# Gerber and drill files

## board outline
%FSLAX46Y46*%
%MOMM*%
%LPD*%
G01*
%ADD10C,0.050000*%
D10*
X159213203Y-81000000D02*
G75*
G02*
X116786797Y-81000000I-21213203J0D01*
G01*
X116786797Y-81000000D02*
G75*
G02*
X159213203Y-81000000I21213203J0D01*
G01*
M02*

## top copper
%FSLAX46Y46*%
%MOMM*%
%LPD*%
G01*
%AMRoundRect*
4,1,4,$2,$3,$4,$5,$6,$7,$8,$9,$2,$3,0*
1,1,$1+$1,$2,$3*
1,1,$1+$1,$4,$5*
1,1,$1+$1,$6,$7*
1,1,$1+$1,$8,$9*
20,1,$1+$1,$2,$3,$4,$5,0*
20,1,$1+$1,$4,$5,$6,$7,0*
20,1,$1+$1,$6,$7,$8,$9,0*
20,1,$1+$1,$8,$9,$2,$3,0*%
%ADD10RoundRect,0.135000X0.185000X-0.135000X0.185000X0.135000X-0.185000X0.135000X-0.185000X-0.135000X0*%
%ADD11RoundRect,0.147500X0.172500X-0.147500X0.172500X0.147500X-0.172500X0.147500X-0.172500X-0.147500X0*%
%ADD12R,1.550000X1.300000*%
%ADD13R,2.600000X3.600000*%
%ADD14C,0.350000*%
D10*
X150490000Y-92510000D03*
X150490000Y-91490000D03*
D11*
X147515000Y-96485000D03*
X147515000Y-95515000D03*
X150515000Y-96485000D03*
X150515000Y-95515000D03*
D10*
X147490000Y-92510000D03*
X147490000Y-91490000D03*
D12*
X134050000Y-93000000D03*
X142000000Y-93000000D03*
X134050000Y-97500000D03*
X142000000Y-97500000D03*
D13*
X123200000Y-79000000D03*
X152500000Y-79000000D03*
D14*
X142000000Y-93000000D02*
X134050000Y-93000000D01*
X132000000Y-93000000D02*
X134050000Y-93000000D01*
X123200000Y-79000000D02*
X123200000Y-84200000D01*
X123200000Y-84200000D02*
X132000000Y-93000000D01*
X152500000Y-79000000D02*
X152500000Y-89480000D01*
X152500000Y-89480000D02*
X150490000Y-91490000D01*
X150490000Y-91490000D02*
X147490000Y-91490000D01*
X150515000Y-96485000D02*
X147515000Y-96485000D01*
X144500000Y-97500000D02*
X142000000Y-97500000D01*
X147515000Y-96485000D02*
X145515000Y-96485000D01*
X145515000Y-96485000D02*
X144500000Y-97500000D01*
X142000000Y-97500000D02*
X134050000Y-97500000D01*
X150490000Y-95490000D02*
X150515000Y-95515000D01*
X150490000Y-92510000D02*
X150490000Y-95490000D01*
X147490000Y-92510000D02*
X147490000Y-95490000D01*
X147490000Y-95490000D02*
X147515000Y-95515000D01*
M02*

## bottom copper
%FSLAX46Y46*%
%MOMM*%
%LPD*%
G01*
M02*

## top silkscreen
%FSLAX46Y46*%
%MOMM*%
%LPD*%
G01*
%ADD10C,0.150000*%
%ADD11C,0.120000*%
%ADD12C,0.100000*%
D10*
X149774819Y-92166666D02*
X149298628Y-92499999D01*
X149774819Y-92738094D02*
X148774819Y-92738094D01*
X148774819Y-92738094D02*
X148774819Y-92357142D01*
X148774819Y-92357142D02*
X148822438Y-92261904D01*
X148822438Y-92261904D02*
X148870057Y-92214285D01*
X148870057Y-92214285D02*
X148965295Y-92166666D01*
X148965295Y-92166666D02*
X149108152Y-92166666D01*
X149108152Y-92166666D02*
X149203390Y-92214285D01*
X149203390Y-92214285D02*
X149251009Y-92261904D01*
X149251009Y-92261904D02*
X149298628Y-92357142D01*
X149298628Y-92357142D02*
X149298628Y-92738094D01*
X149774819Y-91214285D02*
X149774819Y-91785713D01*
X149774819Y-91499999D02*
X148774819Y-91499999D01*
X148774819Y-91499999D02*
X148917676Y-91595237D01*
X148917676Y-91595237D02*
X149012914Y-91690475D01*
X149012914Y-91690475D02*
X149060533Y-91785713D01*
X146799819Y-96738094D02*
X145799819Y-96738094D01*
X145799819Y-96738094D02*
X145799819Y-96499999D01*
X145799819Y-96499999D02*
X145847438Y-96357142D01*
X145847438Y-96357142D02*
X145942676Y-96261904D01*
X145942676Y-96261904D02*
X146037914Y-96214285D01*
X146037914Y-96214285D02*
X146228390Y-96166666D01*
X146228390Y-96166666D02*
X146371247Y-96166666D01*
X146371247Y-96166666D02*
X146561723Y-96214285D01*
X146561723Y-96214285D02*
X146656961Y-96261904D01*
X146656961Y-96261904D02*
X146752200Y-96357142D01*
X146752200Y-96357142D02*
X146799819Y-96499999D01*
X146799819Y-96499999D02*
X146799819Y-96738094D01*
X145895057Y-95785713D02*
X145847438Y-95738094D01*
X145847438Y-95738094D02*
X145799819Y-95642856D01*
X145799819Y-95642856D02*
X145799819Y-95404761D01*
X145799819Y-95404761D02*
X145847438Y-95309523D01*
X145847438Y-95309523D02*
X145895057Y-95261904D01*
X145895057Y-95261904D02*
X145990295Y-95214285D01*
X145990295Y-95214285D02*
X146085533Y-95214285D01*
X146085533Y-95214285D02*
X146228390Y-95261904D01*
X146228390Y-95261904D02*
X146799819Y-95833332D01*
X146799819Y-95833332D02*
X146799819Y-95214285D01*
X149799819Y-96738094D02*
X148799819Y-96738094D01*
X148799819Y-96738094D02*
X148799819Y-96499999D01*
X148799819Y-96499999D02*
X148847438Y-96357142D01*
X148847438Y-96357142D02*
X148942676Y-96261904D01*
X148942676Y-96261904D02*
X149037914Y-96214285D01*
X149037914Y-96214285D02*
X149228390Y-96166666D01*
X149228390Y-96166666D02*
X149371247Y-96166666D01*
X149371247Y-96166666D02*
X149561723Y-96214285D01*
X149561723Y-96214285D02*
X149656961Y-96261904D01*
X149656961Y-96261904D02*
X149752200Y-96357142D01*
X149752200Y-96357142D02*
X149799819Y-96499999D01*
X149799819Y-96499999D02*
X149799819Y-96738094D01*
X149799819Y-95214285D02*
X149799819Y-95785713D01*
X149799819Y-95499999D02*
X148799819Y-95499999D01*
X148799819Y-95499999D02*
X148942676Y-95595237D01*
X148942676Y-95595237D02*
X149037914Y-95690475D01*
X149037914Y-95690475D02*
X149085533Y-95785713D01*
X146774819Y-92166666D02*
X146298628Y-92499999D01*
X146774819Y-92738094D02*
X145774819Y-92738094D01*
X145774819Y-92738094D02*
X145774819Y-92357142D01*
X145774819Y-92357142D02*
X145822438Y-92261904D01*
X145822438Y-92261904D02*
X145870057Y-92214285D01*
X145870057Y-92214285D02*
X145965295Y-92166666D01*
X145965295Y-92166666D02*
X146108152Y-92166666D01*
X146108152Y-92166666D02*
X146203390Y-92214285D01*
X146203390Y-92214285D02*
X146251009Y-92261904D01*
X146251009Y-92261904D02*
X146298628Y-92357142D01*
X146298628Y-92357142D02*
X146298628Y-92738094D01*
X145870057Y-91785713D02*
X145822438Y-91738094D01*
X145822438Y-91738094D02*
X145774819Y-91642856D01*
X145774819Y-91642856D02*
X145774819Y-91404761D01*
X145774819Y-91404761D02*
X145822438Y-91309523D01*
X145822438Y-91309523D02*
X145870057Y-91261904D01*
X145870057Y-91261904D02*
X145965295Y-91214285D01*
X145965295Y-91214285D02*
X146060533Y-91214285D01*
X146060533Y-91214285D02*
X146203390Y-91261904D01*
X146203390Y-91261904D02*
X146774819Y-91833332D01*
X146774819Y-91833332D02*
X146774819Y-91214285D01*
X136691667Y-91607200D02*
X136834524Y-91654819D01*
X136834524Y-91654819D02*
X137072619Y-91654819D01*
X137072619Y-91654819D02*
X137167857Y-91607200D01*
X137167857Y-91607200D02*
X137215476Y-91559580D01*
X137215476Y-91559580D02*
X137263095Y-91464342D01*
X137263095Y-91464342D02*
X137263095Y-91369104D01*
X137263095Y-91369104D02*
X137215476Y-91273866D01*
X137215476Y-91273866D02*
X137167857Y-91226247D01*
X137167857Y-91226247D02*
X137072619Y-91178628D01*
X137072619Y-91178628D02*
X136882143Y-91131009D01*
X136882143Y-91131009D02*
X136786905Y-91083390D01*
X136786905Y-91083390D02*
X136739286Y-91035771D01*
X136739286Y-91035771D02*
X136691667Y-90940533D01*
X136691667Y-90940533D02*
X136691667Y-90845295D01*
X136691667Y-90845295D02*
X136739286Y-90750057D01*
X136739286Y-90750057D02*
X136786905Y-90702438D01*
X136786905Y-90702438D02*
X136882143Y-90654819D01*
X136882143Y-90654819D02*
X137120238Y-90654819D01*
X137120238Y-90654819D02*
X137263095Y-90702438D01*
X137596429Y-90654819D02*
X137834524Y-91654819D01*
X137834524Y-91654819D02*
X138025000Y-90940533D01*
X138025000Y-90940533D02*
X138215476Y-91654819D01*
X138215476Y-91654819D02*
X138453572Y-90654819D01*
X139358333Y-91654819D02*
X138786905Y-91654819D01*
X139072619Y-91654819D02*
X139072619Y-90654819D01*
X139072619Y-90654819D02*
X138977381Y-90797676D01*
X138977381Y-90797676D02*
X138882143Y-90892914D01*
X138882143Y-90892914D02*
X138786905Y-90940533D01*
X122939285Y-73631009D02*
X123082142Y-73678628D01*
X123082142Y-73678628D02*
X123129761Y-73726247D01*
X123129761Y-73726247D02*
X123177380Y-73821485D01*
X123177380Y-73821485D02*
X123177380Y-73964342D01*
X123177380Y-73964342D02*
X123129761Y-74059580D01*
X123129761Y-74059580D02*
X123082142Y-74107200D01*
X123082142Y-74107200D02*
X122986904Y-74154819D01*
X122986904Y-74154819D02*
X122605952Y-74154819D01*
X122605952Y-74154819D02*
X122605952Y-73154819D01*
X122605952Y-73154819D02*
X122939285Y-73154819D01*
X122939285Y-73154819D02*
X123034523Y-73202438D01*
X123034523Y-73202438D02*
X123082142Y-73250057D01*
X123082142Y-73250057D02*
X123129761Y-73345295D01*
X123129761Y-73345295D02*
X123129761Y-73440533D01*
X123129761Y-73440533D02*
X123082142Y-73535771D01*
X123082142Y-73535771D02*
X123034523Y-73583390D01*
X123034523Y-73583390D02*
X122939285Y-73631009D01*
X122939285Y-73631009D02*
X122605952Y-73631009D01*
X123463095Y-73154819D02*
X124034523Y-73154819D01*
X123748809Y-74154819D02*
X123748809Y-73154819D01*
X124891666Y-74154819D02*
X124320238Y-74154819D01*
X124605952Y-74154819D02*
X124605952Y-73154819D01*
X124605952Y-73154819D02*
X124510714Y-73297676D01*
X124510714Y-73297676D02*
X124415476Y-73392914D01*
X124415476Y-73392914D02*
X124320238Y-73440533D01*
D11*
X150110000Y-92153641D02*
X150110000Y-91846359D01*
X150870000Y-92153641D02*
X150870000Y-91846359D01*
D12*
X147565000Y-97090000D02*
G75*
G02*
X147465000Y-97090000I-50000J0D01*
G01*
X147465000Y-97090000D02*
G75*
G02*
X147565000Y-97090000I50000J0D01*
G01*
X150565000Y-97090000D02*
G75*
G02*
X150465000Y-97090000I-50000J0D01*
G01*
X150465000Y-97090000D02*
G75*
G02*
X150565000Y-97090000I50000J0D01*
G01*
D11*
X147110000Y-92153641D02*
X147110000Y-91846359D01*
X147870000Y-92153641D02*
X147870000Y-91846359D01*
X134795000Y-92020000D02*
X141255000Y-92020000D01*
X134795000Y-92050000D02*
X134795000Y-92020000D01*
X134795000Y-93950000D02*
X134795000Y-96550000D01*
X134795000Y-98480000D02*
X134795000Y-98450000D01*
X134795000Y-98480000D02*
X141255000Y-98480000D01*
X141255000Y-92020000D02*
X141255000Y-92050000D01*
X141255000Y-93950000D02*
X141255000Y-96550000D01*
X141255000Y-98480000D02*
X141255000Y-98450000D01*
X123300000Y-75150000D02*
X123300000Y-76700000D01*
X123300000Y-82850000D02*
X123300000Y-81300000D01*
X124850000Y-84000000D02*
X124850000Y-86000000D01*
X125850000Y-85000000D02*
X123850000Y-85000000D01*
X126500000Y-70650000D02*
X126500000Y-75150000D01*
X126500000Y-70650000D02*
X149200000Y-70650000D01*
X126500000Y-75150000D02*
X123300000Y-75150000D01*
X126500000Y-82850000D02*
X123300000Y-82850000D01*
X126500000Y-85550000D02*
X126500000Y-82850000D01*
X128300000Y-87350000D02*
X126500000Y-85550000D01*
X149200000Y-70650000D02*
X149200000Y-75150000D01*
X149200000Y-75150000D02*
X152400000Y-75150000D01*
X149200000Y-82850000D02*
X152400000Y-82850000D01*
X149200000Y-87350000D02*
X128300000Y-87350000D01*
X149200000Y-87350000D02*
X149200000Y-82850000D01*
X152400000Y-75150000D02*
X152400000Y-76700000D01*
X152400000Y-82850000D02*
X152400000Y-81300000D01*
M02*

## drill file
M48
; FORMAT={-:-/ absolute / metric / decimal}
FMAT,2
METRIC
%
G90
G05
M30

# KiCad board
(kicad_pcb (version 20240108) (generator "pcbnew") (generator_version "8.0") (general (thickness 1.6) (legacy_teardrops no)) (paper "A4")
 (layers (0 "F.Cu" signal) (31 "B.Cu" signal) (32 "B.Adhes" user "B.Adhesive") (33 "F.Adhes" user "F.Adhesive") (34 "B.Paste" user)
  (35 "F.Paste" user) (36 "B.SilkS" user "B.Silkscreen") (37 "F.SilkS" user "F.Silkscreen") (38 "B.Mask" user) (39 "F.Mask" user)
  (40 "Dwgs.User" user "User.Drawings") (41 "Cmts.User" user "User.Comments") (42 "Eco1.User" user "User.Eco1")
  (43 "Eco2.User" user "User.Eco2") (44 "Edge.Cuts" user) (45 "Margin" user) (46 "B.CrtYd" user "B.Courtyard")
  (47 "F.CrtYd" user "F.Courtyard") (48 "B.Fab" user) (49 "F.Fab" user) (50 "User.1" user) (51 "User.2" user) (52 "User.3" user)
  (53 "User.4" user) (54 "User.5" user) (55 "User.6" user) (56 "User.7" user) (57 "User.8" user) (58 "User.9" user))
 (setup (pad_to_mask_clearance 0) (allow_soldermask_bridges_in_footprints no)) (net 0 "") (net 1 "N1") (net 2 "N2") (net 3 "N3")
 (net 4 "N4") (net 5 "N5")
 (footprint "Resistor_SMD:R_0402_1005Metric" (layer "F.Cu") (at 150.49 92 90)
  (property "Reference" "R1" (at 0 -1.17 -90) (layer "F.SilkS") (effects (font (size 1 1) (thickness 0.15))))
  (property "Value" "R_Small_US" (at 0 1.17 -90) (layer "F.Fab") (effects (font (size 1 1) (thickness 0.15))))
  (fp_line (start -0.153641 -0.38) (end 0.153641 -0.38) (stroke (width 0.12) (type solid)) (layer "F.SilkS"))
  (fp_line (start -0.153641 0.38) (end 0.153641 0.38) (stroke (width 0.12) (type solid)) (layer "F.SilkS"))
  (pad "1" smd roundrect (at -0.51 0 90) (size 0.54 0.64) (layers "F.Cu" "F.Paste" "F.Mask") (roundrect_rratio 0.25) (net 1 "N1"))
  (pad "2" smd roundrect (at 0.51 0 90) (size 0.54 0.64) (layers "F.Cu" "F.Paste" "F.Mask") (roundrect_rratio 0.25) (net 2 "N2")))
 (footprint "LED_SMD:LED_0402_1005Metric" (layer "F.Cu") (at 147.515 96 90)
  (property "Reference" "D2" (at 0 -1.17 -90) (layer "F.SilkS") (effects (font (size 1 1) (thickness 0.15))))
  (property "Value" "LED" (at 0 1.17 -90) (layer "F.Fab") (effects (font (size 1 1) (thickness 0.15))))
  (fp_circle (center -1.09 0) (end -1.04 0) (stroke (width 0.1) (type solid)) (fill none) (layer "F.SilkS"))
  (pad "1" smd roundrect (at -0.485 0 90) (size 0.59 0.64) (layers "F.Cu" "F.Paste" "F.Mask") (roundrect_rratio 0.25) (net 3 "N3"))
  (pad "2" smd roundrect (at 0.485 0 90) (size 0.59 0.64) (layers "F.Cu" "F.Paste" "F.Mask") (roundrect_rratio 0.25) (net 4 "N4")))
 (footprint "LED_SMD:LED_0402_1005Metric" (layer "F.Cu") (at 150.515 96 90)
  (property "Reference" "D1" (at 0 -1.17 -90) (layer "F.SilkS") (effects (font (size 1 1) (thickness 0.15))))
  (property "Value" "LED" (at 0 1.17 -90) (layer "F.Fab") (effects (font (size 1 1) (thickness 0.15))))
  (fp_circle (center -1.09 0) (end -1.04 0) (stroke (width 0.1) (type solid)) (fill none) (layer "F.SilkS"))
  (pad "1" smd roundrect (at -0.485 0 90) (size 0.59 0.64) (layers "F.Cu" "F.Paste" "F.Mask") (roundrect_rratio 0.25) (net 3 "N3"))
  (pad "2" smd roundrect (at 0.485 0 90) (size 0.59 0.64) (layers "F.Cu" "F.Paste" "F.Mask") (roundrect_rratio 0.25) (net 1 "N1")))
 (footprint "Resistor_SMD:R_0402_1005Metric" (layer "F.Cu") (at 147.49 92 90)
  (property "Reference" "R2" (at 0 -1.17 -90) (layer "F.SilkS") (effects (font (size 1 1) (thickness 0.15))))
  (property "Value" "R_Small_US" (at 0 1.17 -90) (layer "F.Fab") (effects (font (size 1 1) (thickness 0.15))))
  (fp_line (start -0.153641 -0.38) (end 0.153641 -0.38) (stroke (width 0.12) (type solid)) (layer "F.SilkS"))
  (fp_line (start -0.153641 0.38) (end 0.153641 0.38) (stroke (width 0.12) (type solid)) (layer "F.SilkS"))
  (pad "1" smd roundrect (at -0.51 0 90) (size 0.54 0.64) (layers "F.Cu" "F.Paste" "F.Mask") (roundrect_rratio 0.25) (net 4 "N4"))
  (pad "2" smd roundrect (at 0.51 0 90) (size 0.54 0.64) (layers "F.Cu" "F.Paste" "F.Mask") (roundrect_rratio 0.25) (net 2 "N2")))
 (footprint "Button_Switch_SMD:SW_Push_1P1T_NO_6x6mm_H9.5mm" (layer "F.Cu") (at 138.025 95.25)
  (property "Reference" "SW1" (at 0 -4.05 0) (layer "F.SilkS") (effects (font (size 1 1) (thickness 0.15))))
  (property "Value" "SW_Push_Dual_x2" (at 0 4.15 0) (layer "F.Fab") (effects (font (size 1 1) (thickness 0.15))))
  (fp_line (start -3.23 -3.23) (end 3.23 -3.23) (stroke (width 0.12) (type solid)) (layer "F.SilkS"))
  (fp_line (start -3.23 -3.2) (end -3.23 -3.23) (stroke (width 0.12) (type solid)) (layer "F.SilkS"))
  (fp_line (start -3.23 -1.3) (end -3.23 1.3) (stroke (width 0.12) (type solid)) (layer "F.SilkS"))
  (fp_line (start -3.23 3.23) (end -3.23 3.2) (stroke (width 0.12) (type solid)) (layer "F.SilkS"))
  (fp_line (start -3.23 3.23) (end 3.23 3.23) (stroke (width 0.12) (type solid)) (layer "F.SilkS"))
  (fp_line (start 3.23 -3.23) (end 3.23 -3.2) (stroke (width 0.12) (type solid)) (layer "F.SilkS"))
  (fp_line (start 3.23 -1.3) (end 3.23 1.3) (stroke (width 0.12) (type solid)) (layer "F.SilkS"))
  (fp_line (start 3.23 3.23) (end 3.23 3.2) (stroke (width 0.12) (type solid)) (layer "F.SilkS"))
  (pad "1" smd rect (at -3.975 -2.25) (size 1.55 1.3) (layers "F.Cu" "F.Paste" "F.Mask") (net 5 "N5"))
  (pad "1" smd rect (at 3.975 -2.25) (size 1.55 1.3) (layers "F.Cu" "F.Paste" "F.Mask") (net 5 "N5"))
  (pad "2" smd rect (at -3.975 2.25) (size 1.55 1.3) (layers "F.Cu" "F.Paste" "F.Mask") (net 3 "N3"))
  (pad "2" smd rect (at 3.975 2.25) (size 1.55 1.3) (layers "F.Cu" "F.Paste" "F.Mask") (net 3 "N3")))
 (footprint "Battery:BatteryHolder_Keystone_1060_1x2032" (layer "F.Cu") (at 137.85 79)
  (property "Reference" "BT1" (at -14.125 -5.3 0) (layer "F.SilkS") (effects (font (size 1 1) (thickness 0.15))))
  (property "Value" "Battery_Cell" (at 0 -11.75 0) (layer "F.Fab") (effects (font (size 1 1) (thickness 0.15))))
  (fp_line (start -14.55 -3.85) (end -14.55 -2.3) (stroke (width 0.12) (type solid)) (layer "F.SilkS"))
  (fp_line (start -14.55 3.85) (end -14.55 2.3) (stroke (width 0.12) (type solid)) (layer "F.SilkS"))
  (fp_line (start -13 5) (end -13 7) (stroke (width 0.12) (type solid)) (layer "F.SilkS"))
  (fp_line (start -12 6) (end -14 6) (stroke (width 0.12) (type solid)) (layer "F.SilkS"))
  (fp_line (start -11.35 -8.35) (end -11.35 -3.85) (stroke (width 0.12) (type solid)) (layer "F.SilkS"))
  (fp_line (start -11.35 -8.35) (end 11.35 -8.35) (stroke (width 0.12) (type solid)) (layer "F.SilkS"))
  (fp_line (start -11.35 -3.85) (end -14.55 -3.85) (stroke (width 0.12) (type solid)) (layer "F.SilkS"))
  (fp_line (start -11.35 3.85) (end -14.55 3.85) (stroke (width 0.12) (type solid)) (layer "F.SilkS"))
  (fp_line (start -11.35 6.55) (end -11.35 3.85) (stroke (width 0.12) (type solid)) (layer "F.SilkS"))
  (fp_line (start -9.55 8.35) (end -11.35 6.55) (stroke (width 0.12) (type solid)) (layer "F.SilkS"))
  (fp_line (start 11.35 -8.35) (end 11.35 -3.85) (stroke (width 0.12) (type solid)) (layer "F.SilkS"))
  (fp_line (start 11.35 -3.85) (end 14.55 -3.85) (stroke (width 0.12) (type solid)) (layer "F.SilkS"))
  (fp_line (start 11.35 3.85) (end 14.55 3.85) (stroke (width 0.12) (type solid)) (layer "F.SilkS"))
  (fp_line (start 11.35 8.35) (end -9.55 8.35) (stroke (width 0.12) (type solid)) (layer "F.SilkS"))
  (fp_line (start 11.35 8.35) (end 11.35 3.85) (stroke (width 0.12) (type solid)) (layer "F.SilkS"))
  (fp_line (start 14.55 -3.85) (end 14.55 -2.3) (stroke (width 0.12) (type solid)) (layer "F.SilkS"))
  (fp_line (start 14.55 3.85) (end 14.55 2.3) (stroke (width 0.12) (type solid)) (layer "F.SilkS"))
  (pad "1" smd rect (at -14.65 0 180) (size 2.6 3.6) (layers "F.Cu" "F.Paste" "F.Mask") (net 5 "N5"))
  (pad "2" smd rect (at 14.65 0 180) (size 2.6 3.6) (layers "F.Cu" "F.Paste" "F.Mask") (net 2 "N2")))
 (gr_circle (center 138 81) (end 159 84) (stroke (width 0.05) (type default)) (fill none) (layer "Edge.Cuts"))
 (segment (start 142 93) (end 134.05 93) (width 0.35) (layer "F.Cu") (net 5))
 (segment (start 132 93) (end 134.05 93) (width 0.35) (layer "F.Cu") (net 5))
 (segment (start 123.2 79) (end 123.2 84.2) (width 0.35) (layer "F.Cu") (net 5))
 (segment (start 123.2 84.2) (end 132 93) (width 0.35) (layer "F.Cu") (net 5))
 (segment (start 152.5 79) (end 152.5 89.48) (width 0.35) (layer "F.Cu") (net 2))
 (segment (start 152.5 89.48) (end 150.49 91.49) (width 0.35) (layer "F.Cu") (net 2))
 (segment (start 150.49 91.49) (end 147.49 91.49) (width 0.35) (layer "F.Cu") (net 2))
 (segment (start 150.515 96.485) (end 147.515 96.485) (width 0.35) (layer "F.Cu") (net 3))
 (segment (start 144.5 97.5) (end 142 97.5) (width 0.35) (layer "F.Cu") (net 3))
 (segment (start 147.515 96.485) (end 145.515 96.485) (width 0.35) (layer "F.Cu") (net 3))
 (segment (start 145.515 96.485) (end 144.5 97.5) (width 0.35) (layer "F.Cu") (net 3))
 (segment (start 142 97.5) (end 134.05 97.5) (width 0.35) (layer "F.Cu") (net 3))
 (segment (start 150.49 95.49) (end 150.515 95.515) (width 0.35) (layer "F.Cu") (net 1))
 (segment (start 150.49 92.51) (end 150.49 95.49) (width 0.35) (layer "F.Cu") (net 1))
 (segment (start 147.49 92.51) (end 147.49 95.49) (width 0.35) (layer "F.Cu") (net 4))
 (segment (start 147.49 95.49) (end 147.515 95.515) (width 0.35) (layer "F.Cu") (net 4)))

